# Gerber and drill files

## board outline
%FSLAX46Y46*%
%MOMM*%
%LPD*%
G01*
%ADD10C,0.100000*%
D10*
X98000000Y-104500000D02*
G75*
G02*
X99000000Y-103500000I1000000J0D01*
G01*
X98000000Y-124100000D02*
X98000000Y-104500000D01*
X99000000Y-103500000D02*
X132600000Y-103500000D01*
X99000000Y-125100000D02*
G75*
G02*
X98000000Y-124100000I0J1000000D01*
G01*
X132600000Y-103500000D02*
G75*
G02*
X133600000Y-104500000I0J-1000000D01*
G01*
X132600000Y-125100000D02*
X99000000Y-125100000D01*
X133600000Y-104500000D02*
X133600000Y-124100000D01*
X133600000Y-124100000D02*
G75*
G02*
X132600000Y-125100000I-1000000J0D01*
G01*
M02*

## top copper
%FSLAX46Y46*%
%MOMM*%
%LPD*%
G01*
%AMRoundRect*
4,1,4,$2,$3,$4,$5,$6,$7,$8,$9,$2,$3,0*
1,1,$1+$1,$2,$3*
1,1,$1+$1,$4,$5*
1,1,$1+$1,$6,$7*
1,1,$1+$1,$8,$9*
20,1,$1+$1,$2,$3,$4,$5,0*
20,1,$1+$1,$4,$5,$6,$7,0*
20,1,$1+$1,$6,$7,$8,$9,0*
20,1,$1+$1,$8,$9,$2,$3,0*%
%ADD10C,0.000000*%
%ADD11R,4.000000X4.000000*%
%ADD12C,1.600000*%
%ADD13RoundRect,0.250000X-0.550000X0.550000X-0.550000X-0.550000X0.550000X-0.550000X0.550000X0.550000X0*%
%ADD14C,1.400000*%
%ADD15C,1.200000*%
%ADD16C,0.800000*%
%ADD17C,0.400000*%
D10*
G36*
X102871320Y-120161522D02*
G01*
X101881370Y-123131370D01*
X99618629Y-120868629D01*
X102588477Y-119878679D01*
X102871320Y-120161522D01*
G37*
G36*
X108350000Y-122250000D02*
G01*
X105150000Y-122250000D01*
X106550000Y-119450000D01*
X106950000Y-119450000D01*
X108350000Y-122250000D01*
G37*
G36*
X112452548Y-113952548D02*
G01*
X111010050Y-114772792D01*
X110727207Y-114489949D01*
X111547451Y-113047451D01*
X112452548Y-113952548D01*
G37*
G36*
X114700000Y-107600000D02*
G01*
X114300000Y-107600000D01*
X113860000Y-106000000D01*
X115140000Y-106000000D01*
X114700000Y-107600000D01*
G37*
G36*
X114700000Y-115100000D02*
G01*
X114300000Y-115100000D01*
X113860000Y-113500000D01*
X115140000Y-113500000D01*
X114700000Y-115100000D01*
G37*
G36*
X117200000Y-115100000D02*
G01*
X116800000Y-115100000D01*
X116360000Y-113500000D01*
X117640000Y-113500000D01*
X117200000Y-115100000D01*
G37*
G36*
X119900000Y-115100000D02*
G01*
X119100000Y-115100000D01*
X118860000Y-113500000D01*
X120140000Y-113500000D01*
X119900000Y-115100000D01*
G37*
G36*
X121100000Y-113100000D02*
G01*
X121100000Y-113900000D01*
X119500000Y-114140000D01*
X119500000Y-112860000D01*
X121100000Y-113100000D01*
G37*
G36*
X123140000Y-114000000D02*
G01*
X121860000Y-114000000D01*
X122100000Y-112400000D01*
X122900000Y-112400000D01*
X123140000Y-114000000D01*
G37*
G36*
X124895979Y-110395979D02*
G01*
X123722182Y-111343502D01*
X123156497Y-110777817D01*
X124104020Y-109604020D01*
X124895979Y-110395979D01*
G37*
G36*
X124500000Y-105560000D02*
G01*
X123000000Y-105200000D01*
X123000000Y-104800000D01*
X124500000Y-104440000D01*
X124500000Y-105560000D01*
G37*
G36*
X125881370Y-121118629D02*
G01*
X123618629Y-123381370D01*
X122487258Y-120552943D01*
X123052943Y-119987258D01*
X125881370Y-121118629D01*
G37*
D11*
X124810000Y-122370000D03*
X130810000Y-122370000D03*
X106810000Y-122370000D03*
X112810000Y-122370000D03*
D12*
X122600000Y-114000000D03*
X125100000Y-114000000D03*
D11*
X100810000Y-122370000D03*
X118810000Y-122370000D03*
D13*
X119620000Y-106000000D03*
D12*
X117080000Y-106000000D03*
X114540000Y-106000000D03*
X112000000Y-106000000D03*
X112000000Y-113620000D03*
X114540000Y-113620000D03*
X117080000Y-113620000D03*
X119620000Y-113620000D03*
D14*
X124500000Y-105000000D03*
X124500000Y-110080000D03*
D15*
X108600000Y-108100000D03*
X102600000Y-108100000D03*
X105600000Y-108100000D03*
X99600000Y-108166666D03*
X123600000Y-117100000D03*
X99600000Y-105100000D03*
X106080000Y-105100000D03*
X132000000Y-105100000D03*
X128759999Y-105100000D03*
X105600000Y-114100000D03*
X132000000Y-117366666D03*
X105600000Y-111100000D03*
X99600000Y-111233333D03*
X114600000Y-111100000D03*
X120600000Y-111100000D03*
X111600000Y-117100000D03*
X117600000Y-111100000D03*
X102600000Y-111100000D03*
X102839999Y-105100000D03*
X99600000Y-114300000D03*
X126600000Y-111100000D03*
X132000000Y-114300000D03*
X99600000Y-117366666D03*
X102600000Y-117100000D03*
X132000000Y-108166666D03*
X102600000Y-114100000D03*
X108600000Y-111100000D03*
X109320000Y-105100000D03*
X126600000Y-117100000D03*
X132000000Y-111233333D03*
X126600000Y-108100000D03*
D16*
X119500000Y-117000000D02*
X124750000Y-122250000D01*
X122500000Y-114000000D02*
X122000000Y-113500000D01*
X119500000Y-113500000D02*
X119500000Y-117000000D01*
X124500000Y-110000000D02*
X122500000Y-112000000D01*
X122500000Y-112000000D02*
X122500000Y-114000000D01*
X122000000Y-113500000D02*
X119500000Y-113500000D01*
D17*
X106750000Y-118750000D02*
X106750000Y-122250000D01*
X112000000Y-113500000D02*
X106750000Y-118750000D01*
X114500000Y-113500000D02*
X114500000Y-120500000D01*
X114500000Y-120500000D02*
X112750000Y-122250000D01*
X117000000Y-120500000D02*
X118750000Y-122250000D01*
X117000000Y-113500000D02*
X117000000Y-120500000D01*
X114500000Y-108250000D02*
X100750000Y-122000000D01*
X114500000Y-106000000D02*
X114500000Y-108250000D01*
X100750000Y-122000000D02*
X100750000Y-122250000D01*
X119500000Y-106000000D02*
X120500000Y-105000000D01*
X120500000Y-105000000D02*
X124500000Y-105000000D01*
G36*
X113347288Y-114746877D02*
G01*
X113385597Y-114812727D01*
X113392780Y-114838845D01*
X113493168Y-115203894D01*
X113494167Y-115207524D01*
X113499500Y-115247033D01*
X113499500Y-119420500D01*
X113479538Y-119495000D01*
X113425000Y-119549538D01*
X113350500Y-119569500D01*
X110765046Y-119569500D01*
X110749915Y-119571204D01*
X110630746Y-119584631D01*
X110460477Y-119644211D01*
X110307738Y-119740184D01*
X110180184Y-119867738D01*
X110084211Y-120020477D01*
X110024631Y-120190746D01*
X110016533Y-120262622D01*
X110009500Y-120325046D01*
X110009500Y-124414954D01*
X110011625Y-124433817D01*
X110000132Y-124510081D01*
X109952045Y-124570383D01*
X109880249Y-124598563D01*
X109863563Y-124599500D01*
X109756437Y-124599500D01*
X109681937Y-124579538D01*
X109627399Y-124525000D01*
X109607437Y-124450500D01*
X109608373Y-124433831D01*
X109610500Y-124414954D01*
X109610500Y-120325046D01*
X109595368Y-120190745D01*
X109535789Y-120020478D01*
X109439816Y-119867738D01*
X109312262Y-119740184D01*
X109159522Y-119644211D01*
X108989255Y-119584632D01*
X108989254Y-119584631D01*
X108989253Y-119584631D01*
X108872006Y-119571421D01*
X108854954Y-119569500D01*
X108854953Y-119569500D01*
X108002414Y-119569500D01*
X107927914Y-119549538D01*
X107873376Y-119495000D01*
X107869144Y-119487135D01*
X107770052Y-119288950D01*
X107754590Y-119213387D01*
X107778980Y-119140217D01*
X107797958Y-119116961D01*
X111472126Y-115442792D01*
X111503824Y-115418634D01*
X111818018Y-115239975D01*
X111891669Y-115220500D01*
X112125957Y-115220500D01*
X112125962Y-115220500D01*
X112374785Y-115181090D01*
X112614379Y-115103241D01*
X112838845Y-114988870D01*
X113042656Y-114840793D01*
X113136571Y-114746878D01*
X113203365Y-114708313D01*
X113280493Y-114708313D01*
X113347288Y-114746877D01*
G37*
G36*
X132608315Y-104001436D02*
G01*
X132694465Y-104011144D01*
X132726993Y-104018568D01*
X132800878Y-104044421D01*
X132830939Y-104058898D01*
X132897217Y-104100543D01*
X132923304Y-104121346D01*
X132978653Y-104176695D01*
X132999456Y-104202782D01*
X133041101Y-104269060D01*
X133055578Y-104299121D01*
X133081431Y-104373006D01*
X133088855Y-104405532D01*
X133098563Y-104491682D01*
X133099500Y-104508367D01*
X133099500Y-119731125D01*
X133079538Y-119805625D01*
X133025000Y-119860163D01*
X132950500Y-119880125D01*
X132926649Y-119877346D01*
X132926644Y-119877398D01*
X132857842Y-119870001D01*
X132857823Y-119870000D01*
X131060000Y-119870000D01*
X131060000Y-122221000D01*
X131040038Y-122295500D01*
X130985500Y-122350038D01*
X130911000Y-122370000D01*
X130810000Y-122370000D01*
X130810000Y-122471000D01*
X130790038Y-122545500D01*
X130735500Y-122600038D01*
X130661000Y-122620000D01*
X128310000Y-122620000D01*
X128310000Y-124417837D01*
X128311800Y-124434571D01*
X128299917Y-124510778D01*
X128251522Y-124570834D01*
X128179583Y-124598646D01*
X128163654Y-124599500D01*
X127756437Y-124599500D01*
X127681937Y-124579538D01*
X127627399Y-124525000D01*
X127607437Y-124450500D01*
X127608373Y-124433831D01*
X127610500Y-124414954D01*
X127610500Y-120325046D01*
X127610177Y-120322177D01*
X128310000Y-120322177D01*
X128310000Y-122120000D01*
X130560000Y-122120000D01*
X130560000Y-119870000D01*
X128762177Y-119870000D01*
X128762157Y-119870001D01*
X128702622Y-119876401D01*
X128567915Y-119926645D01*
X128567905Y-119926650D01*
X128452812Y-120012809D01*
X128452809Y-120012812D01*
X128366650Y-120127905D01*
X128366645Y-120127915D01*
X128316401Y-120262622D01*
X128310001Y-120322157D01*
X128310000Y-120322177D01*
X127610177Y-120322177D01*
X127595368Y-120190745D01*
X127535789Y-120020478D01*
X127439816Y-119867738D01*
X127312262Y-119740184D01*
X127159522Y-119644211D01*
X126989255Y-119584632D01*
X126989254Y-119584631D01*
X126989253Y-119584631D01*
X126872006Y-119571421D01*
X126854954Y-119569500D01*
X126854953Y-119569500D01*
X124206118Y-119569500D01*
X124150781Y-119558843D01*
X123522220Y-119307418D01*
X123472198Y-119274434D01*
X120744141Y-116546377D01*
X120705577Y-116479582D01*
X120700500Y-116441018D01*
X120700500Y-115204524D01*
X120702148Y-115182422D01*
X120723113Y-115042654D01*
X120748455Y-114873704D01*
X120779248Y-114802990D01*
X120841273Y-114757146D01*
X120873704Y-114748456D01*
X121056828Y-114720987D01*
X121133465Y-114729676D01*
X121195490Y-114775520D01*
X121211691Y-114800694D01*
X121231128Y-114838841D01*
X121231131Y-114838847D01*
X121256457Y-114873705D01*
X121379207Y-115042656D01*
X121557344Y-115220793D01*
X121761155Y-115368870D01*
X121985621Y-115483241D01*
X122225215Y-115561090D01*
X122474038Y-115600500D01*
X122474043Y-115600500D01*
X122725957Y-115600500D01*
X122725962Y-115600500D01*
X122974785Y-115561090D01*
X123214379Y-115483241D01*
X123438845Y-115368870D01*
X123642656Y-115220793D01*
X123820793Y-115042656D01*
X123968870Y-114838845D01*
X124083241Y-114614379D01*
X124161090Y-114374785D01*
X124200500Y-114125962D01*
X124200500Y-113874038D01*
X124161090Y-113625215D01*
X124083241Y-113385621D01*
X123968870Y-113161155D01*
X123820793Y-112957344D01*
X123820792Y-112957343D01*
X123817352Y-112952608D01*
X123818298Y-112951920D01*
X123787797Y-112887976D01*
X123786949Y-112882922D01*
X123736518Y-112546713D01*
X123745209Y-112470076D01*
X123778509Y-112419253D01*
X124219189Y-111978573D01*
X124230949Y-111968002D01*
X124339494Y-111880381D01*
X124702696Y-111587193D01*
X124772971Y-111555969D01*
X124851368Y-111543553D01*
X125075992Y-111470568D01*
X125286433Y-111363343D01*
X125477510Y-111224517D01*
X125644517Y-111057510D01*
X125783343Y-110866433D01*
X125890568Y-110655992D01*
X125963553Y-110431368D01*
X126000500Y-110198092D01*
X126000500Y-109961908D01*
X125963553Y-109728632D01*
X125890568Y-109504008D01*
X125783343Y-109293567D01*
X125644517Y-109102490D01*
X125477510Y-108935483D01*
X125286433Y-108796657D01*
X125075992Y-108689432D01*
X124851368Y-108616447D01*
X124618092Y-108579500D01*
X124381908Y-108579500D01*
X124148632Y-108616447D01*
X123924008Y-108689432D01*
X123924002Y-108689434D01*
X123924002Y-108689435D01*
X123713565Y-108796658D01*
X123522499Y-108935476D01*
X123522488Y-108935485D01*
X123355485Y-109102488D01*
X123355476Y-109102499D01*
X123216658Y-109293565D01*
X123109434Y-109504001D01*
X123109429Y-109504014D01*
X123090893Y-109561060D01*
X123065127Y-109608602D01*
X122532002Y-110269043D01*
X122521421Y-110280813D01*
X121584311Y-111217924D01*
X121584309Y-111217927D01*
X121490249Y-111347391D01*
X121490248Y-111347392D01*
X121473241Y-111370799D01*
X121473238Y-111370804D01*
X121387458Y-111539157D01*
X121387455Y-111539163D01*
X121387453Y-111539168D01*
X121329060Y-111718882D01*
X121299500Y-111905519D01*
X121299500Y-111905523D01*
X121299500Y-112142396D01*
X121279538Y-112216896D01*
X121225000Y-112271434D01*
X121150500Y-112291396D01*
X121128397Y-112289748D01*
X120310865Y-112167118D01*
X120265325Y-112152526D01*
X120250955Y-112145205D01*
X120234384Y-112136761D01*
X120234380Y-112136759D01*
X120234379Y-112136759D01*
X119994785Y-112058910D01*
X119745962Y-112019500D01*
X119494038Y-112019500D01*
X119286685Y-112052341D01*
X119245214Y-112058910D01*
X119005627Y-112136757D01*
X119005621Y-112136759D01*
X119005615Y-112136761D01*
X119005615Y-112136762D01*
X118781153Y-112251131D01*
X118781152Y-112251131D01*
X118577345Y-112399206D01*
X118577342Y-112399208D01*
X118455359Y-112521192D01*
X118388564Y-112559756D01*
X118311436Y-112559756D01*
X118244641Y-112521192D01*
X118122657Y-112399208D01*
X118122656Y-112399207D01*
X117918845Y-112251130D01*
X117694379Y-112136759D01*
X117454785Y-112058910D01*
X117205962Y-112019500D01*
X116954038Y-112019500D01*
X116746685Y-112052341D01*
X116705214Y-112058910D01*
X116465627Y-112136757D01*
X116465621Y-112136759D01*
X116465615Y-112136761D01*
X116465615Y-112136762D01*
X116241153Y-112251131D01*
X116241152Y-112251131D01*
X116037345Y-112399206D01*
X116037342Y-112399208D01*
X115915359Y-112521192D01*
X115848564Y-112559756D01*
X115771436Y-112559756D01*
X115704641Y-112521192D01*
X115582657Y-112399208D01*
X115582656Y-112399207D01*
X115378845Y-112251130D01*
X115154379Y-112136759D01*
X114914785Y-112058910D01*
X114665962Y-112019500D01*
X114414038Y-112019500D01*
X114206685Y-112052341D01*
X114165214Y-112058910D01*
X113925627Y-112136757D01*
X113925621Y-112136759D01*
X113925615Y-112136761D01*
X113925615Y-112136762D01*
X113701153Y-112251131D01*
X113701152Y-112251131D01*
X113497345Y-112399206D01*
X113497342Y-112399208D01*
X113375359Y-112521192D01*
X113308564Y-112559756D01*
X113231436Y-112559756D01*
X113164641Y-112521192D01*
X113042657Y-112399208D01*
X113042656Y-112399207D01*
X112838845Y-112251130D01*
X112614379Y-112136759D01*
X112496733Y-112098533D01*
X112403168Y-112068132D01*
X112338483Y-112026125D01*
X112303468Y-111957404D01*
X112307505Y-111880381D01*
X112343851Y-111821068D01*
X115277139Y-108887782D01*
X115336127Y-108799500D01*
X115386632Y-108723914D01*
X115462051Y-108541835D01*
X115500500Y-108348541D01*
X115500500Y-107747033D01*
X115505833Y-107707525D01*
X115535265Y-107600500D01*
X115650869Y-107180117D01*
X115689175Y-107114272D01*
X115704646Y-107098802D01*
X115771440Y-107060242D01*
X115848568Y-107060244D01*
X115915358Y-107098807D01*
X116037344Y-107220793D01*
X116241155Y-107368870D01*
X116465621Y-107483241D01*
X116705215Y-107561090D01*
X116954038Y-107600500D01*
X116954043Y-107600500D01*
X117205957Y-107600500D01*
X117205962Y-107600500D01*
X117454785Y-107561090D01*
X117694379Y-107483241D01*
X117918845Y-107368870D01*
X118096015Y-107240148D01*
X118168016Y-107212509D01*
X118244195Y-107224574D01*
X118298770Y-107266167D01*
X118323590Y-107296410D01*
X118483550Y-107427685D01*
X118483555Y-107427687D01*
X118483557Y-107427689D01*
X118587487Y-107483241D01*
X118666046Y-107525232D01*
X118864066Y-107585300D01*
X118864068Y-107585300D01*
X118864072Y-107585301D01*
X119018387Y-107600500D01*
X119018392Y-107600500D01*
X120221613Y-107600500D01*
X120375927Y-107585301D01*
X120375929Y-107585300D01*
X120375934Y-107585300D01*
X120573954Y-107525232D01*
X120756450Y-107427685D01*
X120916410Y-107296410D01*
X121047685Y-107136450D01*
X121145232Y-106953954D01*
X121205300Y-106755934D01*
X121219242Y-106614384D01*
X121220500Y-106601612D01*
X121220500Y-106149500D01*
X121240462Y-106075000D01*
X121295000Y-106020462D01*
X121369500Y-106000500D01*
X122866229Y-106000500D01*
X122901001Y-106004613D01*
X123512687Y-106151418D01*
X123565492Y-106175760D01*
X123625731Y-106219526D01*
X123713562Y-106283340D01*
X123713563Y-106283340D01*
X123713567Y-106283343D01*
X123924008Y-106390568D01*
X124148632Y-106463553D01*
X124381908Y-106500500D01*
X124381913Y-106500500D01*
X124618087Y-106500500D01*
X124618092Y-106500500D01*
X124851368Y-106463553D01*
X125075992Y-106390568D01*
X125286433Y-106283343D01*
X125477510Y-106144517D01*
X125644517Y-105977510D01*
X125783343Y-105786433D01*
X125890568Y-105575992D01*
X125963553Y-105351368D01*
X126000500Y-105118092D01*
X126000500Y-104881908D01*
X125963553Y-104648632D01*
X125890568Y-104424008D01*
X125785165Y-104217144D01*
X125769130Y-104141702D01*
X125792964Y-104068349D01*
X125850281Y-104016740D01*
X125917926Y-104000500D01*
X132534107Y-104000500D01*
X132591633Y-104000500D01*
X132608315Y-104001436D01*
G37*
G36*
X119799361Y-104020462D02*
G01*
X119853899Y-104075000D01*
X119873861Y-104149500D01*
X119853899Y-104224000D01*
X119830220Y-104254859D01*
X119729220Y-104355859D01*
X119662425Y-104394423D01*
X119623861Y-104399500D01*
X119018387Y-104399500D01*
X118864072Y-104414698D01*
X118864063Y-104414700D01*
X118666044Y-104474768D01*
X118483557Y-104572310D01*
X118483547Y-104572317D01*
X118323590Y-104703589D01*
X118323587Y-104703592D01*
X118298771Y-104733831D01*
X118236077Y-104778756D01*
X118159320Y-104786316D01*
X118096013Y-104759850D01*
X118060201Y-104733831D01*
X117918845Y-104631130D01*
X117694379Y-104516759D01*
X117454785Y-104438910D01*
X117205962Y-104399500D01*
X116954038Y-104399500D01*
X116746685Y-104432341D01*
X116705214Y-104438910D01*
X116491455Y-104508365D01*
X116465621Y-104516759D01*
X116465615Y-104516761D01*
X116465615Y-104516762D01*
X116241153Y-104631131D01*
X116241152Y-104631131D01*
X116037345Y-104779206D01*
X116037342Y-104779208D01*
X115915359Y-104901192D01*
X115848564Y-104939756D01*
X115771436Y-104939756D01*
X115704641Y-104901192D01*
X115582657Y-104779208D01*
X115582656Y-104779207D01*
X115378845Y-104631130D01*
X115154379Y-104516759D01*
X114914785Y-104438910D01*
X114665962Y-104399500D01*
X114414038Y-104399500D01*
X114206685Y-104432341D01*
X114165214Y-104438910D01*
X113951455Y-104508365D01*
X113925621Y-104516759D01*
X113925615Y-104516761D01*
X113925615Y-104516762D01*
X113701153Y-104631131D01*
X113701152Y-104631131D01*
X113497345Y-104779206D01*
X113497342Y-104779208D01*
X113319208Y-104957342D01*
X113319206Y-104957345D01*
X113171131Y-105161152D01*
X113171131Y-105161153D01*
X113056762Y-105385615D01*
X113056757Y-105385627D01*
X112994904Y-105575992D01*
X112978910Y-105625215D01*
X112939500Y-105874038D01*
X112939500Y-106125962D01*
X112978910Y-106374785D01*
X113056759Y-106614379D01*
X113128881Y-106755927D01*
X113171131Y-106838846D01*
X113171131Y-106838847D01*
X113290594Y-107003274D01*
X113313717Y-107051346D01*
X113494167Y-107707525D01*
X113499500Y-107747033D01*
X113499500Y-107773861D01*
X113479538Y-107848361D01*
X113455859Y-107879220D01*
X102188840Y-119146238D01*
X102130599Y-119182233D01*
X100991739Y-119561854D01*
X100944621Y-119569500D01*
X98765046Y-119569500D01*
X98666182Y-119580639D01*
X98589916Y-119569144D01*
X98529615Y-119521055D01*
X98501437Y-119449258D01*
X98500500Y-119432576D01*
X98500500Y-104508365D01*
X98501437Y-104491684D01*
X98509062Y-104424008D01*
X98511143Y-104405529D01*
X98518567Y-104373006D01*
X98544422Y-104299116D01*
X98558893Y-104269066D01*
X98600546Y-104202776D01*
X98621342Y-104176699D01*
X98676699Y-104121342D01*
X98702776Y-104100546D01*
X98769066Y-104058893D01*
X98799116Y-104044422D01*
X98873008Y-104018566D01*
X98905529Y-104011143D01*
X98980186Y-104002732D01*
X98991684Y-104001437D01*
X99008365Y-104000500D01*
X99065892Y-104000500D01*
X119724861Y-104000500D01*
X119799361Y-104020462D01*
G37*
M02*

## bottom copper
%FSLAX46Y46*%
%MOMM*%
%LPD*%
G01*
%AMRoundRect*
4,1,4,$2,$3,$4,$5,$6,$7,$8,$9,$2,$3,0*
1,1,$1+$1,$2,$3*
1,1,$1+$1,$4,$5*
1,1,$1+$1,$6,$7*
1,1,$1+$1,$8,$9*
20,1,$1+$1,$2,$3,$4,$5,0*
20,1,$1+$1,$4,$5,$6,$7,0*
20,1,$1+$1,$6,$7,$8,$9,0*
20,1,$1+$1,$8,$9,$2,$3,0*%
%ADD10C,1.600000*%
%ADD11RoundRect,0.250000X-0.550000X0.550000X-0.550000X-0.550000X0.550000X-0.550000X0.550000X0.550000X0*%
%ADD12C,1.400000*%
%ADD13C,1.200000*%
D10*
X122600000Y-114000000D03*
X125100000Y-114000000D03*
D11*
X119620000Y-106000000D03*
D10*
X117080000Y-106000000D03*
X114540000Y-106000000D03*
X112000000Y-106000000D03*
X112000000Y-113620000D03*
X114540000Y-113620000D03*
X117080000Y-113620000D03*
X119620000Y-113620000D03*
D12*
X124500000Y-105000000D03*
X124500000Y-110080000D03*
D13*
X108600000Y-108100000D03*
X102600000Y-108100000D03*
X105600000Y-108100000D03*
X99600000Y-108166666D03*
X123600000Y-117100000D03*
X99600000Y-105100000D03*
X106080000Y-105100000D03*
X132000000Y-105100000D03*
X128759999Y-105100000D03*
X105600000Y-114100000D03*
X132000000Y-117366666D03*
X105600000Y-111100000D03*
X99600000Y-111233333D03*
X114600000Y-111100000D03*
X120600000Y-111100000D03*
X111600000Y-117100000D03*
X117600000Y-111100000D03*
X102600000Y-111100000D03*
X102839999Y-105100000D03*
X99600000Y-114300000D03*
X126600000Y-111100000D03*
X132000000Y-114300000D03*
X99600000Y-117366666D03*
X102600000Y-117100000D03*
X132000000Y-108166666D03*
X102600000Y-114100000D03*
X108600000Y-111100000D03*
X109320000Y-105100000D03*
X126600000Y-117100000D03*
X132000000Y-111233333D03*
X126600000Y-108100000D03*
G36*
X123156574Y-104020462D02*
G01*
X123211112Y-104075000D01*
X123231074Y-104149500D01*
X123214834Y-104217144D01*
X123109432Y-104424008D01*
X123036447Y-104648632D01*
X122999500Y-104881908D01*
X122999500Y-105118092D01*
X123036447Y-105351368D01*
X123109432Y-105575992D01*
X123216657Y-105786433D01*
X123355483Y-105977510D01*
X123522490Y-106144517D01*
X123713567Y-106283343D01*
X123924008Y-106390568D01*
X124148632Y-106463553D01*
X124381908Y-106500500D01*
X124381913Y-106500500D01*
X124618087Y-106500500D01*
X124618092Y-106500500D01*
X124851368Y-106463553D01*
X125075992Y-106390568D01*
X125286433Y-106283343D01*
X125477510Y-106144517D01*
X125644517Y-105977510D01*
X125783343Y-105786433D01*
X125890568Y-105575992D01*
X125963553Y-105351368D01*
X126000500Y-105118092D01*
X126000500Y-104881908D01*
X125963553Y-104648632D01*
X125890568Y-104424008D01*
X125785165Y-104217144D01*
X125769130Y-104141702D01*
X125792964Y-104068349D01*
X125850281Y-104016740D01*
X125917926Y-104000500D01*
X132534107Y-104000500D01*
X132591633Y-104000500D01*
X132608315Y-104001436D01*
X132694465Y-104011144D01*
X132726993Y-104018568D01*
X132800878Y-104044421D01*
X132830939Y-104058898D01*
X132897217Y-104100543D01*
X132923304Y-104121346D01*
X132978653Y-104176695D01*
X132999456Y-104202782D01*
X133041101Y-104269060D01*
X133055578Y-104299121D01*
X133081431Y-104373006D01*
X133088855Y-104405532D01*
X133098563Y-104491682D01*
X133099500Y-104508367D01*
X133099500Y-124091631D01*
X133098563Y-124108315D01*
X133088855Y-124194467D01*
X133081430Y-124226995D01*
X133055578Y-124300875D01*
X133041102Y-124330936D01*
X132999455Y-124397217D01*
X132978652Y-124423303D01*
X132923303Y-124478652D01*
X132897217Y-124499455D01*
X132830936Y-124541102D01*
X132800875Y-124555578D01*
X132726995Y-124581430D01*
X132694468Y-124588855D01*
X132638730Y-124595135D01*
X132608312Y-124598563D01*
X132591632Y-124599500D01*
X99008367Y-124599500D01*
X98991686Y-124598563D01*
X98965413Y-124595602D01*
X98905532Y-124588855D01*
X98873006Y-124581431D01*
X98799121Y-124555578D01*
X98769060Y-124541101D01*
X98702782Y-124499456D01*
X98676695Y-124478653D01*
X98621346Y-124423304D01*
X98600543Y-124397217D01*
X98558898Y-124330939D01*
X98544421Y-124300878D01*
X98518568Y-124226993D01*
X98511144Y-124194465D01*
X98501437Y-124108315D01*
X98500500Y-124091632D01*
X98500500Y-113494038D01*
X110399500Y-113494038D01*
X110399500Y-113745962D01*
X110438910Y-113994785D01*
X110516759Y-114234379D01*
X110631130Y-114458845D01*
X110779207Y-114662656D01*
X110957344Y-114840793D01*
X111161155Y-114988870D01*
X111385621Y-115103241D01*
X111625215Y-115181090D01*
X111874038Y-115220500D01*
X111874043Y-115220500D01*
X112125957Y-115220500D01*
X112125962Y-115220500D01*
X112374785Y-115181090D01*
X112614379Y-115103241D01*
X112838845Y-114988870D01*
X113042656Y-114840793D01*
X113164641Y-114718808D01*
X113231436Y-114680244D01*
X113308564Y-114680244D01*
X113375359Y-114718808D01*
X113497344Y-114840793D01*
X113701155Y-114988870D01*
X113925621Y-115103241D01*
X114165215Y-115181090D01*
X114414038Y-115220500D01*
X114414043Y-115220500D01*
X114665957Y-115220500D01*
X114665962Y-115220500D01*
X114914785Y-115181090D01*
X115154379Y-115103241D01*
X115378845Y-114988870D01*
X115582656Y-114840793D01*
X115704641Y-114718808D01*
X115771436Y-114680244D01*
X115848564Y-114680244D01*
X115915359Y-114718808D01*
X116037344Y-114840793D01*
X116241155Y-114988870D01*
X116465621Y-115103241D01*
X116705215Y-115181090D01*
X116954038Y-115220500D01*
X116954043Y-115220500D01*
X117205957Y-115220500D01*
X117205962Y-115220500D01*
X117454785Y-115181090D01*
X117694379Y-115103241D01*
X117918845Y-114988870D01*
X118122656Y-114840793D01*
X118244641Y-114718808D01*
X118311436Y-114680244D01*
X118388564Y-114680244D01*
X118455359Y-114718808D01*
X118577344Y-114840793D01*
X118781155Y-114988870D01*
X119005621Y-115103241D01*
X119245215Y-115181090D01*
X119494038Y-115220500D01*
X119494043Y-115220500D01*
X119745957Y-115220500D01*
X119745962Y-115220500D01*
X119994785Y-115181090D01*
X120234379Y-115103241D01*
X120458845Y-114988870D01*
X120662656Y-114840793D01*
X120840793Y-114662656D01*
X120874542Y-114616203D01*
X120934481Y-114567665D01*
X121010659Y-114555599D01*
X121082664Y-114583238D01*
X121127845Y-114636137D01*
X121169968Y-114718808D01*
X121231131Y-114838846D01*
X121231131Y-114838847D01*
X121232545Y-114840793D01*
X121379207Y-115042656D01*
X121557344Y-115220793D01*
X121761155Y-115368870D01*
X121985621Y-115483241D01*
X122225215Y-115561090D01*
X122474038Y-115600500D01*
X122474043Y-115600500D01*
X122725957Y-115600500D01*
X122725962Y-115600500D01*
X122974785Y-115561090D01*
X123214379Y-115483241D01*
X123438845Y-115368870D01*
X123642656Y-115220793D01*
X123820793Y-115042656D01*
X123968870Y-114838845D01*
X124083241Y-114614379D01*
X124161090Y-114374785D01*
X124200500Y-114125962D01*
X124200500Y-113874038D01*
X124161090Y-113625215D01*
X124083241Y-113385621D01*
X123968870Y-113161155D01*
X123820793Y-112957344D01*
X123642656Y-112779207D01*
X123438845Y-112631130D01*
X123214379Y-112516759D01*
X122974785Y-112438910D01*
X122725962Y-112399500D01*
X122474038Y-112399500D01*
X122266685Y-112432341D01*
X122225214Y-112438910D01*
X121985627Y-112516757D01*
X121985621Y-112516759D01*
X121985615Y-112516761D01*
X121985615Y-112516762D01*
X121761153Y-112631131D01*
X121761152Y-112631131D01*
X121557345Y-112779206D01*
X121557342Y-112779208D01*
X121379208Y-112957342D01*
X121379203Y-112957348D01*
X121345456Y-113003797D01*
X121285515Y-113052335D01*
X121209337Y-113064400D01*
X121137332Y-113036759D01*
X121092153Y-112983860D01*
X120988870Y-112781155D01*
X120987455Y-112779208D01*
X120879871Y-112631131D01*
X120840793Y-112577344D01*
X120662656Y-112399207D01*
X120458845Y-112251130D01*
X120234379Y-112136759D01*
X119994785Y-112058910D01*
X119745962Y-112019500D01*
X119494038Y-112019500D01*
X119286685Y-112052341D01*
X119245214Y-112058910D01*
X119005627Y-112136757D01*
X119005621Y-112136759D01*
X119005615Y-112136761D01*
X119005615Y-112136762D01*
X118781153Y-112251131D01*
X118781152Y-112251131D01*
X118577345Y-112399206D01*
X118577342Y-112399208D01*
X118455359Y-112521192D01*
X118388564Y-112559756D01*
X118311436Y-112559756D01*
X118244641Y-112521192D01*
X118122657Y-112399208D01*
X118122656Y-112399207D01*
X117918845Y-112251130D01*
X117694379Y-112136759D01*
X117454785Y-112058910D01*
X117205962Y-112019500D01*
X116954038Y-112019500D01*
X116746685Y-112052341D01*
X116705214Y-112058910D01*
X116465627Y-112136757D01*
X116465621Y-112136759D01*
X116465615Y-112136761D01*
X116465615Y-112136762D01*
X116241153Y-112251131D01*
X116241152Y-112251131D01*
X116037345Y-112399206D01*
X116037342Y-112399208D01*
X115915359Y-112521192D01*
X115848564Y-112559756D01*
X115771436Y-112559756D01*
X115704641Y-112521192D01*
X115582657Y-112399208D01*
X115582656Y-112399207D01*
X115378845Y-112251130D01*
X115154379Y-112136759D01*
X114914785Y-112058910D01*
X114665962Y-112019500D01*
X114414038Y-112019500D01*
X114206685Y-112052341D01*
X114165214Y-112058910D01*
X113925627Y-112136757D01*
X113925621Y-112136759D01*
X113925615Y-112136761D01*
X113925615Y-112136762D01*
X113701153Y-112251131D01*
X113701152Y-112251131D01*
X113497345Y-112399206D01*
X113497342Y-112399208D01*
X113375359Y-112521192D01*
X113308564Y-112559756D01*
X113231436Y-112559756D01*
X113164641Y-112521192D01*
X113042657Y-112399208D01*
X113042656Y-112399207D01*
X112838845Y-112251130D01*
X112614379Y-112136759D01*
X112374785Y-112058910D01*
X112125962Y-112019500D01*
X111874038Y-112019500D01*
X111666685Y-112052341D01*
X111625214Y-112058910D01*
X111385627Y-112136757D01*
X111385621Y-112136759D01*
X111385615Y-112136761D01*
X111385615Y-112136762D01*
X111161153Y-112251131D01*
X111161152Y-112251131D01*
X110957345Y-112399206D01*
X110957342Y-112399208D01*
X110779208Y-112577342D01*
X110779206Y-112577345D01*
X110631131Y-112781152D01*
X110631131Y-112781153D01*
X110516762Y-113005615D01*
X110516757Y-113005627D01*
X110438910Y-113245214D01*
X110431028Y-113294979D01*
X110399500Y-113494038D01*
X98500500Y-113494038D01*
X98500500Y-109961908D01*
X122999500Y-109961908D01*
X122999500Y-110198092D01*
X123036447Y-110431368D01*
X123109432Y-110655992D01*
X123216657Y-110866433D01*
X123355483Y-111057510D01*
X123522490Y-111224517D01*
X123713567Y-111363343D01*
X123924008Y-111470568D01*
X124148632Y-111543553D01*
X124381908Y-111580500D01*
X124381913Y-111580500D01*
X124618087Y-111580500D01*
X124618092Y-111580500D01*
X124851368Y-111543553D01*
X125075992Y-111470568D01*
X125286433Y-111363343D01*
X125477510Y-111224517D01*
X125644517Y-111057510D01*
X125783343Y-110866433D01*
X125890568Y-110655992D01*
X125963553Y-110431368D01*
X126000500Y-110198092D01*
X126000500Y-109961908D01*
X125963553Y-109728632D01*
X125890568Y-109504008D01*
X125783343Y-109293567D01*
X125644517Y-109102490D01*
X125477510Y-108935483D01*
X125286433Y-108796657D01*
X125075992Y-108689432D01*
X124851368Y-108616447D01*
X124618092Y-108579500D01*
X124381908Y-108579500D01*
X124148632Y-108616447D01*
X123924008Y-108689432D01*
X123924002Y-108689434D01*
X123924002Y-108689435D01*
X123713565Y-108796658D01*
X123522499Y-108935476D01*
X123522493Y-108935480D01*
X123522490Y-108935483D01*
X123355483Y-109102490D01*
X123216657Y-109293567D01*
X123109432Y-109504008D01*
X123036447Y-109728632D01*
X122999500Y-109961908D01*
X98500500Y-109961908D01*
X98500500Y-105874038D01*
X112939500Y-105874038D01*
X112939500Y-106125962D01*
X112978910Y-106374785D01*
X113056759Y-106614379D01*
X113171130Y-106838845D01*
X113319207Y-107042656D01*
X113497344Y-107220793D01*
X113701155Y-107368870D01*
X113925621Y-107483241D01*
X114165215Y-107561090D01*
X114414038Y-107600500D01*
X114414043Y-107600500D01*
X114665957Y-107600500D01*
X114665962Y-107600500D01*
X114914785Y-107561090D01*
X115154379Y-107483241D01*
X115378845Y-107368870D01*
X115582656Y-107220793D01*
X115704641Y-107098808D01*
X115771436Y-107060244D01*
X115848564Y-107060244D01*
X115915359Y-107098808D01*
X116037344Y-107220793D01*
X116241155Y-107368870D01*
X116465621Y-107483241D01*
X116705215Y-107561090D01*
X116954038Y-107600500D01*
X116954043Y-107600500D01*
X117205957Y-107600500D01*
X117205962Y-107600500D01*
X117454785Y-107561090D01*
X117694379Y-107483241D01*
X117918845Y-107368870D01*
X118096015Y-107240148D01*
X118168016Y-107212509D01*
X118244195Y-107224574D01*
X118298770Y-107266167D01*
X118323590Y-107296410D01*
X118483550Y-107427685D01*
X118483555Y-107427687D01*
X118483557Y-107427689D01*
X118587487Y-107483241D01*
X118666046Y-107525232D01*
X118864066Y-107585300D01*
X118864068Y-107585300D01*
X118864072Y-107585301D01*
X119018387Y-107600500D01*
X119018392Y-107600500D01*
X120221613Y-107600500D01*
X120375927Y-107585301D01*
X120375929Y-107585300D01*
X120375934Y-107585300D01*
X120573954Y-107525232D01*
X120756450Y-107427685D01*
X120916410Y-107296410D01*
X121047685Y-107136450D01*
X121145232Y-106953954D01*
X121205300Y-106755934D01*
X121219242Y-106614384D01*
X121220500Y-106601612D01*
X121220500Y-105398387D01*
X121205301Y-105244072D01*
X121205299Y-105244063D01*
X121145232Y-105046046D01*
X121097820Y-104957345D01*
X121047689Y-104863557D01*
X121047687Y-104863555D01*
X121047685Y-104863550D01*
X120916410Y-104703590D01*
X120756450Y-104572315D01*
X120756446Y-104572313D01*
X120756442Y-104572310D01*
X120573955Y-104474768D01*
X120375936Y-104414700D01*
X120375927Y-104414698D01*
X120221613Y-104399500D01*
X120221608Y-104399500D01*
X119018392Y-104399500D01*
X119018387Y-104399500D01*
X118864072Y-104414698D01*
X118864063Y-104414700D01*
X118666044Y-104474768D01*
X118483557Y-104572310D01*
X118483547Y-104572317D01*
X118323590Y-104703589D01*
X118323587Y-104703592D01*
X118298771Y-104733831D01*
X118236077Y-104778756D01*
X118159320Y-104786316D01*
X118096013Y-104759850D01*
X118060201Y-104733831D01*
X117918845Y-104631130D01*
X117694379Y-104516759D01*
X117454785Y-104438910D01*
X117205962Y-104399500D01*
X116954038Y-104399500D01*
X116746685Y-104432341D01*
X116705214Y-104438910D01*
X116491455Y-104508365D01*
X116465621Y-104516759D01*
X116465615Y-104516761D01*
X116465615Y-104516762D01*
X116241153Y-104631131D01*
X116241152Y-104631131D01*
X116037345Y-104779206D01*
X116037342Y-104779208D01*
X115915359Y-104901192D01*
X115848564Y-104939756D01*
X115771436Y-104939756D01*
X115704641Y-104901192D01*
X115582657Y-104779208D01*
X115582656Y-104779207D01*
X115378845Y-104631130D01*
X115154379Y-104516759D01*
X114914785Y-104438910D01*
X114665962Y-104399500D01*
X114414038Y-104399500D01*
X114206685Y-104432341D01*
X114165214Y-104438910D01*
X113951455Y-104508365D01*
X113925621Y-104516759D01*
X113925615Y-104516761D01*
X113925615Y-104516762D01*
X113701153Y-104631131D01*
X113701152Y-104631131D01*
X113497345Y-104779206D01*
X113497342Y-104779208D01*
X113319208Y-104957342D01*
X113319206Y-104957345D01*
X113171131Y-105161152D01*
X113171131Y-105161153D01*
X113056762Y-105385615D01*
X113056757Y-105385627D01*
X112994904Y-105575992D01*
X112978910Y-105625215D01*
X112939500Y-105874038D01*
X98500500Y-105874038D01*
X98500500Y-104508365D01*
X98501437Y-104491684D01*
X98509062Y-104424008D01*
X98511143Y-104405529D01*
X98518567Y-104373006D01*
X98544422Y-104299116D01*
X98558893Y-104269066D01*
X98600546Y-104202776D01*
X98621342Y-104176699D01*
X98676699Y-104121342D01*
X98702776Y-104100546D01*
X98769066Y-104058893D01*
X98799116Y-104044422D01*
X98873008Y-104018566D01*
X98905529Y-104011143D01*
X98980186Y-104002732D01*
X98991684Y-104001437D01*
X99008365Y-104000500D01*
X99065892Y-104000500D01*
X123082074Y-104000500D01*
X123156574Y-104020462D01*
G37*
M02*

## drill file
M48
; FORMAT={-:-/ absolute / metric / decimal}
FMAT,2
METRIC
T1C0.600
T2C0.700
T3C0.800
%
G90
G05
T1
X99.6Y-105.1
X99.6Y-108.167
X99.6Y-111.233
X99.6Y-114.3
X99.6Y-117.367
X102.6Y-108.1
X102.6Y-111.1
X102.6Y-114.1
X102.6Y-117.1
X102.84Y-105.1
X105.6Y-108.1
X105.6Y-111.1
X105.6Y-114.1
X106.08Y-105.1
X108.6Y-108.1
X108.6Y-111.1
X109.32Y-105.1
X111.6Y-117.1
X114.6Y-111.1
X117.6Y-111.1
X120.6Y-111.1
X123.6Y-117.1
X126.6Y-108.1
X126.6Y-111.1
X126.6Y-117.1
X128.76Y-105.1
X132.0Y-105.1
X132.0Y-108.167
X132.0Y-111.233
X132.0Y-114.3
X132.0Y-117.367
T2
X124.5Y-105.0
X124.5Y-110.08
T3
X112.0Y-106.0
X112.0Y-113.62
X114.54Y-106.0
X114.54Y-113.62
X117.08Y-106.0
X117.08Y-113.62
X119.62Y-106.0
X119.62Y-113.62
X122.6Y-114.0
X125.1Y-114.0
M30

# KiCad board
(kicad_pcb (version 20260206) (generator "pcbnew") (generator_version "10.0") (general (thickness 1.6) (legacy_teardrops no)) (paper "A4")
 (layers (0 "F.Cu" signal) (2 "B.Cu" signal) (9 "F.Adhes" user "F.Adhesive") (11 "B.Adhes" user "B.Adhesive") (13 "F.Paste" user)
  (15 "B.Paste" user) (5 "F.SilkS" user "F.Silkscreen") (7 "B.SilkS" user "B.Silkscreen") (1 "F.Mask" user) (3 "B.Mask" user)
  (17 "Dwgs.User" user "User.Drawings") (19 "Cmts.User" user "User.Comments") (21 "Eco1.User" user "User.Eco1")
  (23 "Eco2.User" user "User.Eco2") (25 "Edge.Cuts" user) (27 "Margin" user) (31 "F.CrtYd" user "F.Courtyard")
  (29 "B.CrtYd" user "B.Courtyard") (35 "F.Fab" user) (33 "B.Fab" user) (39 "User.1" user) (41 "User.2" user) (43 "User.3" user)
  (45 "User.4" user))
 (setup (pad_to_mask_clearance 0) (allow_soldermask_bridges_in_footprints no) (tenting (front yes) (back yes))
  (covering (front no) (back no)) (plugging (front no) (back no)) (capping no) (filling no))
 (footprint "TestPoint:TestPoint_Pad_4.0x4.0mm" (layer "F.Cu") (at 124.81 122.37)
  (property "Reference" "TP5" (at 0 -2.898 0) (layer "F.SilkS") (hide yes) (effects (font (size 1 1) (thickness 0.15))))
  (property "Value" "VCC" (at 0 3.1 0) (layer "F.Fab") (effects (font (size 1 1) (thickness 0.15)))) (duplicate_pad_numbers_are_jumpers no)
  (pad "1" smd rect (at 0 0) (size 4 4) (layers "F.Cu" "F.Mask") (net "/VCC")))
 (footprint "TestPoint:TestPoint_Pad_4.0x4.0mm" (layer "F.Cu") (at 130.81 122.37)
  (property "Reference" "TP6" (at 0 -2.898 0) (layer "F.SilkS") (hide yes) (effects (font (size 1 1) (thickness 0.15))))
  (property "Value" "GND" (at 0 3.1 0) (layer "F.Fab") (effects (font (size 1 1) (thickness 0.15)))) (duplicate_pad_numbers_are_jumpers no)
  (pad "1" smd rect (at 0 0) (size 4 4) (layers "F.Cu" "F.Mask") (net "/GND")))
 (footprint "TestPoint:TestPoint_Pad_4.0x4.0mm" (layer "F.Cu") (at 106.81 122.37)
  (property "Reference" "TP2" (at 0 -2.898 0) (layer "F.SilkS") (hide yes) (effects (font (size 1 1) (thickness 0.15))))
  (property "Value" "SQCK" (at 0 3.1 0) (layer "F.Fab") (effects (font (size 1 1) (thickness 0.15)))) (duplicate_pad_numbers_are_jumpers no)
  (pad "1" smd rect (at 0 0) (size 4 4) (layers "F.Cu" "F.Mask") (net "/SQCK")))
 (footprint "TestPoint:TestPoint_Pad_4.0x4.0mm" (layer "F.Cu") (at 112.81 122.37)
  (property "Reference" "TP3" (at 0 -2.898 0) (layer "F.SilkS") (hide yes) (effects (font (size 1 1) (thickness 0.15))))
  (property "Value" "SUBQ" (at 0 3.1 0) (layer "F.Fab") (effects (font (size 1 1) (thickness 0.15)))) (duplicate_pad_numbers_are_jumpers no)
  (pad "1" smd rect (at 0 0) (size 4 4) (layers "F.Cu" "F.Mask") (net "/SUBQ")))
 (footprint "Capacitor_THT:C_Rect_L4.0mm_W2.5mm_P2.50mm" (layer "F.Cu") (at 122.6 114)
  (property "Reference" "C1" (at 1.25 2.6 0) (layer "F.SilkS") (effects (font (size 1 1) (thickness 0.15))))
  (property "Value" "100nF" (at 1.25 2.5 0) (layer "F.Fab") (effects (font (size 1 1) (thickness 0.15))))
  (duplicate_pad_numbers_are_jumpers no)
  (pad "1" thru_hole circle (at 0 0) (size 1.6 1.6) (drill 0.8) (layers "*.Cu" "*.Mask") (remove_unused_layers no) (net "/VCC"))
  (pad "2" thru_hole circle (at 2.5 0) (size 1.6 1.6) (drill 0.8) (layers "*.Cu" "*.Mask") (remove_unused_layers no) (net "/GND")
   (zone_connect 2)))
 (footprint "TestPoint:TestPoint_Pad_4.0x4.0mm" (layer "F.Cu") (at 100.81 122.37)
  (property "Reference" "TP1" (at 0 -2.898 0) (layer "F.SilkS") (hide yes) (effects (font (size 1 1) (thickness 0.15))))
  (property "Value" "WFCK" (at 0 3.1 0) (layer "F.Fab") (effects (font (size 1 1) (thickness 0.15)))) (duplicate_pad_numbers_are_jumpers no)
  (pad "1" smd rect (at 0 0) (size 4 4) (layers "F.Cu" "F.Mask") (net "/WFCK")))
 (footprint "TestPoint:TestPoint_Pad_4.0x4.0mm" (layer "F.Cu") (at 118.81 122.37)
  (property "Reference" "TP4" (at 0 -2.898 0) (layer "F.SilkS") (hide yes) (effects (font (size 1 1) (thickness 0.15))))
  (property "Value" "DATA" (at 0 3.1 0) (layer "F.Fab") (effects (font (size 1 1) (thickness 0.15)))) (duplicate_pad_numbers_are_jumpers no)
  (pad "1" smd rect (at 0 0) (size 4 4) (layers "F.Cu" "F.Mask") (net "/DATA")))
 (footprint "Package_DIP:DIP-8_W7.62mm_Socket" (layer "F.Cu") (at 119.62 106 -90)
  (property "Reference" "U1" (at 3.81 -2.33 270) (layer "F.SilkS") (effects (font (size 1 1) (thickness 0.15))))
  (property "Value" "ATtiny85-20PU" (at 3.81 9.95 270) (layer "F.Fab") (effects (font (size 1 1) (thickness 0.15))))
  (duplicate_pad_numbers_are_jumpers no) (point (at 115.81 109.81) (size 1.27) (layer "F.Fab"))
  (pad "1" thru_hole roundrect (at 0 0 270) (size 1.6 1.6) (drill 0.8) (layers "*.Cu" "*.Mask") (remove_unused_layers no)
   (roundrect_rratio 0.15625) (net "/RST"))
  (pad "2" thru_hole circle (at 0 2.54 270) (size 1.6 1.6) (drill 0.8) (layers "*.Cu" "*.Mask") (remove_unused_layers no)
   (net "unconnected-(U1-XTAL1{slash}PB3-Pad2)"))
  (pad "3" thru_hole circle (at 0 5.08 270) (size 1.6 1.6) (drill 0.8) (layers "*.Cu" "*.Mask") (remove_unused_layers no) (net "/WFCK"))
  (pad "4" thru_hole circle (at 0 7.62 270) (size 1.6 1.6) (drill 0.8) (layers "*.Cu" "*.Mask") (remove_unused_layers no) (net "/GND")
   (zone_connect 2))
  (pad "5" thru_hole circle (at 7.62 7.62 270) (size 1.6 1.6) (drill 0.8) (layers "*.Cu" "*.Mask") (remove_unused_layers no) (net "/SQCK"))
  (pad "6" thru_hole circle (at 7.62 5.08 270) (size 1.6 1.6) (drill 0.8) (layers "*.Cu" "*.Mask") (remove_unused_layers no) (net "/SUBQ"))
  (pad "7" thru_hole circle (at 7.62 2.54 270) (size 1.6 1.6) (drill 0.8) (layers "*.Cu" "*.Mask") (remove_unused_layers no) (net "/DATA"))
  (pad "8" thru_hole circle (at 7.62 0 270) (size 1.6 1.6) (drill 0.8) (layers "*.Cu" "*.Mask") (remove_unused_layers no) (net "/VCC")))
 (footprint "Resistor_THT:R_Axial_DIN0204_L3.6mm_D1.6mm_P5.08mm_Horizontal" (layer "F.Cu") (at 124.5 105 -90)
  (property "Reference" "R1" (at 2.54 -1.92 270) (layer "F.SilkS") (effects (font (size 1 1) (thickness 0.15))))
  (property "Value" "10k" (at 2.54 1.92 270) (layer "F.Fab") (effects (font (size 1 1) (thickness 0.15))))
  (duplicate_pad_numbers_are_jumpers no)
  (pad "1" thru_hole circle (at 0 0 270) (size 1.4 1.4) (drill 0.7) (layers "*.Cu" "*.Mask") (remove_unused_layers no) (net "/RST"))
  (pad "2" thru_hole circle (at 5.08 0 270) (size 1.4 1.4) (drill 0.7) (layers "*.Cu" "*.Mask") (remove_unused_layers no) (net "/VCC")))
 (gr_poly
  (pts (xy 101.88137 123.13137) (xy 102.87132 120.161522) (xy 102.588477 119.878679) (xy 99.618629 120.868629))
  (stroke (width 0) (type default)) (fill yes) (layer "F.Cu") (net "/WFCK"))
 (gr_poly
  (pts (xy 108.35 122.25) (xy 106.95 119.45) (xy 106.55 119.45) (xy 105.15 122.25)) (stroke (width 0) (type default)) (fill yes)
  (layer "F.Cu") (net "/SQCK"))
 (gr_poly
  (pts (xy 111.547451 113.047451) (xy 110.727207 114.489949) (xy 111.01005 114.772792) (xy 112.452548 113.952548))
  (stroke (width 0) (type default)) (fill yes) (layer "F.Cu") (net "/SQCK"))
 (gr_poly
  (pts (xy 113.86 106) (xy 114.3 107.6) (xy 114.7 107.6) (xy 115.14 106)) (stroke (width 0) (type default)) (fill yes) (layer "F.Cu")
  (net "/WFCK"))
 (gr_poly
  (pts (xy 113.86 113.5) (xy 114.3 115.1) (xy 114.7 115.1) (xy 115.14 113.5)) (stroke (width 0) (type default)) (fill yes) (layer "F.Cu")
  (net "/SUBQ"))
 (gr_poly
  (pts (xy 116.36 113.5) (xy 116.8 115.1) (xy 117.2 115.1) (xy 117.64 113.5)) (stroke (width 0) (type default)) (fill yes) (layer "F.Cu")
  (net "/DATA"))
 (gr_poly
  (pts (xy 118.86 113.5) (xy 119.1 115.1) (xy 119.9 115.1) (xy 120.14 113.5)) (stroke (width 0) (type default)) (fill yes) (layer "F.Cu")
  (net "/VCC"))
 (gr_poly
  (pts (xy 119.5 114.14) (xy 121.1 113.9) (xy 121.1 113.1) (xy 119.5 112.86)) (stroke (width 0) (type default)) (fill yes) (layer "F.Cu")
  (net "/VCC"))
 (gr_poly
  (pts (xy 123.14 114) (xy 122.9 112.4) (xy 122.1 112.4) (xy 121.86 114)) (stroke (width 0) (type default)) (fill yes) (layer "F.Cu")
  (net "/VCC"))
 (gr_poly
  (pts (xy 124.10402 109.60402) (xy 123.156497 110.777817) (xy 123.722182 111.343502) (xy 124.895979 110.395979))
  (stroke (width 0) (type default)) (fill yes) (layer "F.Cu") (net "/VCC"))
 (gr_poly
  (pts (xy 124.5 104.44) (xy 123 104.8) (xy 123 105.2) (xy 124.5 105.56)) (stroke (width 0) (type default)) (fill yes) (layer "F.Cu")
  (net "/RST"))
 (gr_poly
  (pts (xy 125.88137 121.118629) (xy 123.052943 119.987258) (xy 122.487258 120.552943) (xy 123.618629 123.38137))
  (stroke (width 0) (type default)) (fill yes) (layer "F.Cu") (net "/VCC"))
 (gr_arc (start 98 104.5) (mid 98.292893 103.792893) (end 99 103.5) (stroke (width 0.1) (type default)) (layer "Edge.Cuts"))
 (gr_line (start 98 124.1) (end 98 104.5) (stroke (width 0.1) (type default)) (layer "Edge.Cuts"))
 (gr_line (start 99 103.5) (end 132.6 103.5) (stroke (width 0.1) (type default)) (layer "Edge.Cuts"))
 (gr_arc (start 99 125.1) (mid 98.292893 124.807106) (end 98 124.1) (stroke (width 0.1) (type default)) (layer "Edge.Cuts"))
 (gr_arc (start 132.6 103.5) (mid 133.307106 103.792893) (end 133.6 104.5) (stroke (width 0.1) (type default)) (layer "Edge.Cuts"))
 (gr_line (start 132.6 125.1) (end 99 125.1) (stroke (width 0.1) (type default)) (layer "Edge.Cuts"))
 (gr_line (start 133.6 104.5) (end 133.6 124.1) (stroke (width 0.1) (type default)) (layer "Edge.Cuts"))
 (gr_arc (start 133.6 124.1) (mid 133.307106 124.807106) (end 132.6 125.1) (stroke (width 0.1) (type default)) (layer "Edge.Cuts"))
 (segment (start 119.5 117) (end 124.75 122.25) (width 0.8) (layer "F.Cu") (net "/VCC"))
 (segment (start 122.5 114) (end 122 113.5) (width 0.8) (layer "F.Cu") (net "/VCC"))
 (segment (start 119.5 113.5) (end 119.5 117) (width 0.8) (layer "F.Cu") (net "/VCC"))
 (segment (start 124.5 110) (end 122.5 112) (width 0.8) (layer "F.Cu") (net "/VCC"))
 (segment (start 122.5 112) (end 122.5 114) (width 0.8) (layer "F.Cu") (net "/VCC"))
 (segment (start 122 113.5) (end 119.5 113.5) (width 0.8) (layer "F.Cu") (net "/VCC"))
 (via (at 108.6 108.1) (size 1.2) (drill 0.6) (layers "F.Cu" "B.Cu") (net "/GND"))
 (via (at 102.6 108.1) (size 1.2) (drill 0.6) (layers "F.Cu" "B.Cu") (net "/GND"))
 (via (at 105.6 108.1) (size 1.2) (drill 0.6) (layers "F.Cu" "B.Cu") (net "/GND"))
 (via (at 99.6 108.166666) (size 1.2) (drill 0.6) (layers "F.Cu" "B.Cu") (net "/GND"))
 (via (at 123.6 117.1) (size 1.2) (drill 0.6) (layers "F.Cu" "B.Cu") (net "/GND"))
 (via (at 99.6 105.1) (size 1.2) (drill 0.6) (layers "F.Cu" "B.Cu") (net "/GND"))
 (via (at 106.08 105.1) (size 1.2) (drill 0.6) (layers "F.Cu" "B.Cu") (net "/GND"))
 (via (at 132 105.1) (size 1.2) (drill 0.6) (layers "F.Cu" "B.Cu") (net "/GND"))
 (via (at 128.759999 105.1) (size 1.2) (drill 0.6) (layers "F.Cu" "B.Cu") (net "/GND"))
 (via (at 105.6 114.1) (size 1.2) (drill 0.6) (layers "F.Cu" "B.Cu") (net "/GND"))
 (via (at 132 117.366666) (size 1.2) (drill 0.6) (layers "F.Cu" "B.Cu") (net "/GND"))
 (via (at 105.6 111.1) (size 1.2) (drill 0.6) (layers "F.Cu" "B.Cu") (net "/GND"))
 (via (at 99.6 111.233333) (size 1.2) (drill 0.6) (layers "F.Cu" "B.Cu") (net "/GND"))
 (via (at 114.6 111.1) (size 1.2) (drill 0.6) (layers "F.Cu" "B.Cu") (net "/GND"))
 (via (at 120.6 111.1) (size 1.2) (drill 0.6) (layers "F.Cu" "B.Cu") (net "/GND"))
 (via (at 111.6 117.1) (size 1.2) (drill 0.6) (layers "F.Cu" "B.Cu") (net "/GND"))
 (via (at 117.6 111.1) (size 1.2) (drill 0.6) (layers "F.Cu" "B.Cu") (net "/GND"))
 (via (at 102.6 111.1) (size 1.2) (drill 0.6) (layers "F.Cu" "B.Cu") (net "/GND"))
 (via (at 102.839999 105.1) (size 1.2) (drill 0.6) (layers "F.Cu" "B.Cu") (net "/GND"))
 (via (at 99.6 114.3) (size 1.2) (drill 0.6) (layers "F.Cu" "B.Cu") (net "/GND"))
 (via (at 126.6 111.1) (size 1.2) (drill 0.6) (layers "F.Cu" "B.Cu") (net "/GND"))
 (via (at 132 114.3) (size 1.2) (drill 0.6) (layers "F.Cu" "B.Cu") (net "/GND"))
 (via (at 99.6 117.366666) (size 1.2) (drill 0.6) (layers "F.Cu" "B.Cu") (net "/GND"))
 (via (at 102.6 117.1) (size 1.2) (drill 0.6) (layers "F.Cu" "B.Cu") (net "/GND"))
 (via (at 132 108.166666) (size 1.2) (drill 0.6) (layers "F.Cu" "B.Cu") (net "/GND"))
 (via (at 102.6 114.1) (size 1.2) (drill 0.6) (layers "F.Cu" "B.Cu") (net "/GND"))
 (via (at 108.6 111.1) (size 1.2) (drill 0.6) (layers "F.Cu" "B.Cu") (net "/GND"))
 (via (at 109.32 105.1) (size 1.2) (drill 0.6) (layers "F.Cu" "B.Cu") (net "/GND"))
 (via (at 126.6 117.1) (size 1.2) (drill 0.6) (layers "F.Cu" "B.Cu") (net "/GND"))
 (via (at 132 111.233333) (size 1.2) (drill 0.6) (layers "F.Cu" "B.Cu") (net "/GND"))
 (via (at 126.6 108.1) (size 1.2) (drill 0.6) (layers "F.Cu" "B.Cu") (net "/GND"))
 (segment (start 106.75 118.75) (end 106.75 122.25) (width 0.4) (layer "F.Cu") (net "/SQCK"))
 (segment (start 112 113.5) (end 106.75 118.75) (width 0.4) (layer "F.Cu") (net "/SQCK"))
 (segment (start 114.5 113.5) (end 114.5 120.5) (width 0.4) (layer "F.Cu") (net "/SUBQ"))
 (segment (start 114.5 120.5) (end 112.75 122.25) (width 0.4) (layer "F.Cu") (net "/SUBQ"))
 (segment (start 117 120.5) (end 118.75 122.25) (width 0.4) (layer "F.Cu") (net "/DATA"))
 (segment (start 117 113.5) (end 117 120.5) (width 0.4) (layer "F.Cu") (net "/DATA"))
 (segment (start 114.5 108.25) (end 100.75 122) (width 0.4) (layer "F.Cu") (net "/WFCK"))
 (segment (start 114.5 106) (end 114.5 108.25) (width 0.4) (layer "F.Cu") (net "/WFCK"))
 (segment (start 100.75 122) (end 100.75 122.25) (width 0.4) (layer "F.Cu") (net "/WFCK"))
 (segment (start 119.5 106) (end 120.5 105) (width 0.4) (layer "F.Cu") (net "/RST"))
 (segment (start 120.5 105) (end 124.5 105) (width 0.4) (layer "F.Cu") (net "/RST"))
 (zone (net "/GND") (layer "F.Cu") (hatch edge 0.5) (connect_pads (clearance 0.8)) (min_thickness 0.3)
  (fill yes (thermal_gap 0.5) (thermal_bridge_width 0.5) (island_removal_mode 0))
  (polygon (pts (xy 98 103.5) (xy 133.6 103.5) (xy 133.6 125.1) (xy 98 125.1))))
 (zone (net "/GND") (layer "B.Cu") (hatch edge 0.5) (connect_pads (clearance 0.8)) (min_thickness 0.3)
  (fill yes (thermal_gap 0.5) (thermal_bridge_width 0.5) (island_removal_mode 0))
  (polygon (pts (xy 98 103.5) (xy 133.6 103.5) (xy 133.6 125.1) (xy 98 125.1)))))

